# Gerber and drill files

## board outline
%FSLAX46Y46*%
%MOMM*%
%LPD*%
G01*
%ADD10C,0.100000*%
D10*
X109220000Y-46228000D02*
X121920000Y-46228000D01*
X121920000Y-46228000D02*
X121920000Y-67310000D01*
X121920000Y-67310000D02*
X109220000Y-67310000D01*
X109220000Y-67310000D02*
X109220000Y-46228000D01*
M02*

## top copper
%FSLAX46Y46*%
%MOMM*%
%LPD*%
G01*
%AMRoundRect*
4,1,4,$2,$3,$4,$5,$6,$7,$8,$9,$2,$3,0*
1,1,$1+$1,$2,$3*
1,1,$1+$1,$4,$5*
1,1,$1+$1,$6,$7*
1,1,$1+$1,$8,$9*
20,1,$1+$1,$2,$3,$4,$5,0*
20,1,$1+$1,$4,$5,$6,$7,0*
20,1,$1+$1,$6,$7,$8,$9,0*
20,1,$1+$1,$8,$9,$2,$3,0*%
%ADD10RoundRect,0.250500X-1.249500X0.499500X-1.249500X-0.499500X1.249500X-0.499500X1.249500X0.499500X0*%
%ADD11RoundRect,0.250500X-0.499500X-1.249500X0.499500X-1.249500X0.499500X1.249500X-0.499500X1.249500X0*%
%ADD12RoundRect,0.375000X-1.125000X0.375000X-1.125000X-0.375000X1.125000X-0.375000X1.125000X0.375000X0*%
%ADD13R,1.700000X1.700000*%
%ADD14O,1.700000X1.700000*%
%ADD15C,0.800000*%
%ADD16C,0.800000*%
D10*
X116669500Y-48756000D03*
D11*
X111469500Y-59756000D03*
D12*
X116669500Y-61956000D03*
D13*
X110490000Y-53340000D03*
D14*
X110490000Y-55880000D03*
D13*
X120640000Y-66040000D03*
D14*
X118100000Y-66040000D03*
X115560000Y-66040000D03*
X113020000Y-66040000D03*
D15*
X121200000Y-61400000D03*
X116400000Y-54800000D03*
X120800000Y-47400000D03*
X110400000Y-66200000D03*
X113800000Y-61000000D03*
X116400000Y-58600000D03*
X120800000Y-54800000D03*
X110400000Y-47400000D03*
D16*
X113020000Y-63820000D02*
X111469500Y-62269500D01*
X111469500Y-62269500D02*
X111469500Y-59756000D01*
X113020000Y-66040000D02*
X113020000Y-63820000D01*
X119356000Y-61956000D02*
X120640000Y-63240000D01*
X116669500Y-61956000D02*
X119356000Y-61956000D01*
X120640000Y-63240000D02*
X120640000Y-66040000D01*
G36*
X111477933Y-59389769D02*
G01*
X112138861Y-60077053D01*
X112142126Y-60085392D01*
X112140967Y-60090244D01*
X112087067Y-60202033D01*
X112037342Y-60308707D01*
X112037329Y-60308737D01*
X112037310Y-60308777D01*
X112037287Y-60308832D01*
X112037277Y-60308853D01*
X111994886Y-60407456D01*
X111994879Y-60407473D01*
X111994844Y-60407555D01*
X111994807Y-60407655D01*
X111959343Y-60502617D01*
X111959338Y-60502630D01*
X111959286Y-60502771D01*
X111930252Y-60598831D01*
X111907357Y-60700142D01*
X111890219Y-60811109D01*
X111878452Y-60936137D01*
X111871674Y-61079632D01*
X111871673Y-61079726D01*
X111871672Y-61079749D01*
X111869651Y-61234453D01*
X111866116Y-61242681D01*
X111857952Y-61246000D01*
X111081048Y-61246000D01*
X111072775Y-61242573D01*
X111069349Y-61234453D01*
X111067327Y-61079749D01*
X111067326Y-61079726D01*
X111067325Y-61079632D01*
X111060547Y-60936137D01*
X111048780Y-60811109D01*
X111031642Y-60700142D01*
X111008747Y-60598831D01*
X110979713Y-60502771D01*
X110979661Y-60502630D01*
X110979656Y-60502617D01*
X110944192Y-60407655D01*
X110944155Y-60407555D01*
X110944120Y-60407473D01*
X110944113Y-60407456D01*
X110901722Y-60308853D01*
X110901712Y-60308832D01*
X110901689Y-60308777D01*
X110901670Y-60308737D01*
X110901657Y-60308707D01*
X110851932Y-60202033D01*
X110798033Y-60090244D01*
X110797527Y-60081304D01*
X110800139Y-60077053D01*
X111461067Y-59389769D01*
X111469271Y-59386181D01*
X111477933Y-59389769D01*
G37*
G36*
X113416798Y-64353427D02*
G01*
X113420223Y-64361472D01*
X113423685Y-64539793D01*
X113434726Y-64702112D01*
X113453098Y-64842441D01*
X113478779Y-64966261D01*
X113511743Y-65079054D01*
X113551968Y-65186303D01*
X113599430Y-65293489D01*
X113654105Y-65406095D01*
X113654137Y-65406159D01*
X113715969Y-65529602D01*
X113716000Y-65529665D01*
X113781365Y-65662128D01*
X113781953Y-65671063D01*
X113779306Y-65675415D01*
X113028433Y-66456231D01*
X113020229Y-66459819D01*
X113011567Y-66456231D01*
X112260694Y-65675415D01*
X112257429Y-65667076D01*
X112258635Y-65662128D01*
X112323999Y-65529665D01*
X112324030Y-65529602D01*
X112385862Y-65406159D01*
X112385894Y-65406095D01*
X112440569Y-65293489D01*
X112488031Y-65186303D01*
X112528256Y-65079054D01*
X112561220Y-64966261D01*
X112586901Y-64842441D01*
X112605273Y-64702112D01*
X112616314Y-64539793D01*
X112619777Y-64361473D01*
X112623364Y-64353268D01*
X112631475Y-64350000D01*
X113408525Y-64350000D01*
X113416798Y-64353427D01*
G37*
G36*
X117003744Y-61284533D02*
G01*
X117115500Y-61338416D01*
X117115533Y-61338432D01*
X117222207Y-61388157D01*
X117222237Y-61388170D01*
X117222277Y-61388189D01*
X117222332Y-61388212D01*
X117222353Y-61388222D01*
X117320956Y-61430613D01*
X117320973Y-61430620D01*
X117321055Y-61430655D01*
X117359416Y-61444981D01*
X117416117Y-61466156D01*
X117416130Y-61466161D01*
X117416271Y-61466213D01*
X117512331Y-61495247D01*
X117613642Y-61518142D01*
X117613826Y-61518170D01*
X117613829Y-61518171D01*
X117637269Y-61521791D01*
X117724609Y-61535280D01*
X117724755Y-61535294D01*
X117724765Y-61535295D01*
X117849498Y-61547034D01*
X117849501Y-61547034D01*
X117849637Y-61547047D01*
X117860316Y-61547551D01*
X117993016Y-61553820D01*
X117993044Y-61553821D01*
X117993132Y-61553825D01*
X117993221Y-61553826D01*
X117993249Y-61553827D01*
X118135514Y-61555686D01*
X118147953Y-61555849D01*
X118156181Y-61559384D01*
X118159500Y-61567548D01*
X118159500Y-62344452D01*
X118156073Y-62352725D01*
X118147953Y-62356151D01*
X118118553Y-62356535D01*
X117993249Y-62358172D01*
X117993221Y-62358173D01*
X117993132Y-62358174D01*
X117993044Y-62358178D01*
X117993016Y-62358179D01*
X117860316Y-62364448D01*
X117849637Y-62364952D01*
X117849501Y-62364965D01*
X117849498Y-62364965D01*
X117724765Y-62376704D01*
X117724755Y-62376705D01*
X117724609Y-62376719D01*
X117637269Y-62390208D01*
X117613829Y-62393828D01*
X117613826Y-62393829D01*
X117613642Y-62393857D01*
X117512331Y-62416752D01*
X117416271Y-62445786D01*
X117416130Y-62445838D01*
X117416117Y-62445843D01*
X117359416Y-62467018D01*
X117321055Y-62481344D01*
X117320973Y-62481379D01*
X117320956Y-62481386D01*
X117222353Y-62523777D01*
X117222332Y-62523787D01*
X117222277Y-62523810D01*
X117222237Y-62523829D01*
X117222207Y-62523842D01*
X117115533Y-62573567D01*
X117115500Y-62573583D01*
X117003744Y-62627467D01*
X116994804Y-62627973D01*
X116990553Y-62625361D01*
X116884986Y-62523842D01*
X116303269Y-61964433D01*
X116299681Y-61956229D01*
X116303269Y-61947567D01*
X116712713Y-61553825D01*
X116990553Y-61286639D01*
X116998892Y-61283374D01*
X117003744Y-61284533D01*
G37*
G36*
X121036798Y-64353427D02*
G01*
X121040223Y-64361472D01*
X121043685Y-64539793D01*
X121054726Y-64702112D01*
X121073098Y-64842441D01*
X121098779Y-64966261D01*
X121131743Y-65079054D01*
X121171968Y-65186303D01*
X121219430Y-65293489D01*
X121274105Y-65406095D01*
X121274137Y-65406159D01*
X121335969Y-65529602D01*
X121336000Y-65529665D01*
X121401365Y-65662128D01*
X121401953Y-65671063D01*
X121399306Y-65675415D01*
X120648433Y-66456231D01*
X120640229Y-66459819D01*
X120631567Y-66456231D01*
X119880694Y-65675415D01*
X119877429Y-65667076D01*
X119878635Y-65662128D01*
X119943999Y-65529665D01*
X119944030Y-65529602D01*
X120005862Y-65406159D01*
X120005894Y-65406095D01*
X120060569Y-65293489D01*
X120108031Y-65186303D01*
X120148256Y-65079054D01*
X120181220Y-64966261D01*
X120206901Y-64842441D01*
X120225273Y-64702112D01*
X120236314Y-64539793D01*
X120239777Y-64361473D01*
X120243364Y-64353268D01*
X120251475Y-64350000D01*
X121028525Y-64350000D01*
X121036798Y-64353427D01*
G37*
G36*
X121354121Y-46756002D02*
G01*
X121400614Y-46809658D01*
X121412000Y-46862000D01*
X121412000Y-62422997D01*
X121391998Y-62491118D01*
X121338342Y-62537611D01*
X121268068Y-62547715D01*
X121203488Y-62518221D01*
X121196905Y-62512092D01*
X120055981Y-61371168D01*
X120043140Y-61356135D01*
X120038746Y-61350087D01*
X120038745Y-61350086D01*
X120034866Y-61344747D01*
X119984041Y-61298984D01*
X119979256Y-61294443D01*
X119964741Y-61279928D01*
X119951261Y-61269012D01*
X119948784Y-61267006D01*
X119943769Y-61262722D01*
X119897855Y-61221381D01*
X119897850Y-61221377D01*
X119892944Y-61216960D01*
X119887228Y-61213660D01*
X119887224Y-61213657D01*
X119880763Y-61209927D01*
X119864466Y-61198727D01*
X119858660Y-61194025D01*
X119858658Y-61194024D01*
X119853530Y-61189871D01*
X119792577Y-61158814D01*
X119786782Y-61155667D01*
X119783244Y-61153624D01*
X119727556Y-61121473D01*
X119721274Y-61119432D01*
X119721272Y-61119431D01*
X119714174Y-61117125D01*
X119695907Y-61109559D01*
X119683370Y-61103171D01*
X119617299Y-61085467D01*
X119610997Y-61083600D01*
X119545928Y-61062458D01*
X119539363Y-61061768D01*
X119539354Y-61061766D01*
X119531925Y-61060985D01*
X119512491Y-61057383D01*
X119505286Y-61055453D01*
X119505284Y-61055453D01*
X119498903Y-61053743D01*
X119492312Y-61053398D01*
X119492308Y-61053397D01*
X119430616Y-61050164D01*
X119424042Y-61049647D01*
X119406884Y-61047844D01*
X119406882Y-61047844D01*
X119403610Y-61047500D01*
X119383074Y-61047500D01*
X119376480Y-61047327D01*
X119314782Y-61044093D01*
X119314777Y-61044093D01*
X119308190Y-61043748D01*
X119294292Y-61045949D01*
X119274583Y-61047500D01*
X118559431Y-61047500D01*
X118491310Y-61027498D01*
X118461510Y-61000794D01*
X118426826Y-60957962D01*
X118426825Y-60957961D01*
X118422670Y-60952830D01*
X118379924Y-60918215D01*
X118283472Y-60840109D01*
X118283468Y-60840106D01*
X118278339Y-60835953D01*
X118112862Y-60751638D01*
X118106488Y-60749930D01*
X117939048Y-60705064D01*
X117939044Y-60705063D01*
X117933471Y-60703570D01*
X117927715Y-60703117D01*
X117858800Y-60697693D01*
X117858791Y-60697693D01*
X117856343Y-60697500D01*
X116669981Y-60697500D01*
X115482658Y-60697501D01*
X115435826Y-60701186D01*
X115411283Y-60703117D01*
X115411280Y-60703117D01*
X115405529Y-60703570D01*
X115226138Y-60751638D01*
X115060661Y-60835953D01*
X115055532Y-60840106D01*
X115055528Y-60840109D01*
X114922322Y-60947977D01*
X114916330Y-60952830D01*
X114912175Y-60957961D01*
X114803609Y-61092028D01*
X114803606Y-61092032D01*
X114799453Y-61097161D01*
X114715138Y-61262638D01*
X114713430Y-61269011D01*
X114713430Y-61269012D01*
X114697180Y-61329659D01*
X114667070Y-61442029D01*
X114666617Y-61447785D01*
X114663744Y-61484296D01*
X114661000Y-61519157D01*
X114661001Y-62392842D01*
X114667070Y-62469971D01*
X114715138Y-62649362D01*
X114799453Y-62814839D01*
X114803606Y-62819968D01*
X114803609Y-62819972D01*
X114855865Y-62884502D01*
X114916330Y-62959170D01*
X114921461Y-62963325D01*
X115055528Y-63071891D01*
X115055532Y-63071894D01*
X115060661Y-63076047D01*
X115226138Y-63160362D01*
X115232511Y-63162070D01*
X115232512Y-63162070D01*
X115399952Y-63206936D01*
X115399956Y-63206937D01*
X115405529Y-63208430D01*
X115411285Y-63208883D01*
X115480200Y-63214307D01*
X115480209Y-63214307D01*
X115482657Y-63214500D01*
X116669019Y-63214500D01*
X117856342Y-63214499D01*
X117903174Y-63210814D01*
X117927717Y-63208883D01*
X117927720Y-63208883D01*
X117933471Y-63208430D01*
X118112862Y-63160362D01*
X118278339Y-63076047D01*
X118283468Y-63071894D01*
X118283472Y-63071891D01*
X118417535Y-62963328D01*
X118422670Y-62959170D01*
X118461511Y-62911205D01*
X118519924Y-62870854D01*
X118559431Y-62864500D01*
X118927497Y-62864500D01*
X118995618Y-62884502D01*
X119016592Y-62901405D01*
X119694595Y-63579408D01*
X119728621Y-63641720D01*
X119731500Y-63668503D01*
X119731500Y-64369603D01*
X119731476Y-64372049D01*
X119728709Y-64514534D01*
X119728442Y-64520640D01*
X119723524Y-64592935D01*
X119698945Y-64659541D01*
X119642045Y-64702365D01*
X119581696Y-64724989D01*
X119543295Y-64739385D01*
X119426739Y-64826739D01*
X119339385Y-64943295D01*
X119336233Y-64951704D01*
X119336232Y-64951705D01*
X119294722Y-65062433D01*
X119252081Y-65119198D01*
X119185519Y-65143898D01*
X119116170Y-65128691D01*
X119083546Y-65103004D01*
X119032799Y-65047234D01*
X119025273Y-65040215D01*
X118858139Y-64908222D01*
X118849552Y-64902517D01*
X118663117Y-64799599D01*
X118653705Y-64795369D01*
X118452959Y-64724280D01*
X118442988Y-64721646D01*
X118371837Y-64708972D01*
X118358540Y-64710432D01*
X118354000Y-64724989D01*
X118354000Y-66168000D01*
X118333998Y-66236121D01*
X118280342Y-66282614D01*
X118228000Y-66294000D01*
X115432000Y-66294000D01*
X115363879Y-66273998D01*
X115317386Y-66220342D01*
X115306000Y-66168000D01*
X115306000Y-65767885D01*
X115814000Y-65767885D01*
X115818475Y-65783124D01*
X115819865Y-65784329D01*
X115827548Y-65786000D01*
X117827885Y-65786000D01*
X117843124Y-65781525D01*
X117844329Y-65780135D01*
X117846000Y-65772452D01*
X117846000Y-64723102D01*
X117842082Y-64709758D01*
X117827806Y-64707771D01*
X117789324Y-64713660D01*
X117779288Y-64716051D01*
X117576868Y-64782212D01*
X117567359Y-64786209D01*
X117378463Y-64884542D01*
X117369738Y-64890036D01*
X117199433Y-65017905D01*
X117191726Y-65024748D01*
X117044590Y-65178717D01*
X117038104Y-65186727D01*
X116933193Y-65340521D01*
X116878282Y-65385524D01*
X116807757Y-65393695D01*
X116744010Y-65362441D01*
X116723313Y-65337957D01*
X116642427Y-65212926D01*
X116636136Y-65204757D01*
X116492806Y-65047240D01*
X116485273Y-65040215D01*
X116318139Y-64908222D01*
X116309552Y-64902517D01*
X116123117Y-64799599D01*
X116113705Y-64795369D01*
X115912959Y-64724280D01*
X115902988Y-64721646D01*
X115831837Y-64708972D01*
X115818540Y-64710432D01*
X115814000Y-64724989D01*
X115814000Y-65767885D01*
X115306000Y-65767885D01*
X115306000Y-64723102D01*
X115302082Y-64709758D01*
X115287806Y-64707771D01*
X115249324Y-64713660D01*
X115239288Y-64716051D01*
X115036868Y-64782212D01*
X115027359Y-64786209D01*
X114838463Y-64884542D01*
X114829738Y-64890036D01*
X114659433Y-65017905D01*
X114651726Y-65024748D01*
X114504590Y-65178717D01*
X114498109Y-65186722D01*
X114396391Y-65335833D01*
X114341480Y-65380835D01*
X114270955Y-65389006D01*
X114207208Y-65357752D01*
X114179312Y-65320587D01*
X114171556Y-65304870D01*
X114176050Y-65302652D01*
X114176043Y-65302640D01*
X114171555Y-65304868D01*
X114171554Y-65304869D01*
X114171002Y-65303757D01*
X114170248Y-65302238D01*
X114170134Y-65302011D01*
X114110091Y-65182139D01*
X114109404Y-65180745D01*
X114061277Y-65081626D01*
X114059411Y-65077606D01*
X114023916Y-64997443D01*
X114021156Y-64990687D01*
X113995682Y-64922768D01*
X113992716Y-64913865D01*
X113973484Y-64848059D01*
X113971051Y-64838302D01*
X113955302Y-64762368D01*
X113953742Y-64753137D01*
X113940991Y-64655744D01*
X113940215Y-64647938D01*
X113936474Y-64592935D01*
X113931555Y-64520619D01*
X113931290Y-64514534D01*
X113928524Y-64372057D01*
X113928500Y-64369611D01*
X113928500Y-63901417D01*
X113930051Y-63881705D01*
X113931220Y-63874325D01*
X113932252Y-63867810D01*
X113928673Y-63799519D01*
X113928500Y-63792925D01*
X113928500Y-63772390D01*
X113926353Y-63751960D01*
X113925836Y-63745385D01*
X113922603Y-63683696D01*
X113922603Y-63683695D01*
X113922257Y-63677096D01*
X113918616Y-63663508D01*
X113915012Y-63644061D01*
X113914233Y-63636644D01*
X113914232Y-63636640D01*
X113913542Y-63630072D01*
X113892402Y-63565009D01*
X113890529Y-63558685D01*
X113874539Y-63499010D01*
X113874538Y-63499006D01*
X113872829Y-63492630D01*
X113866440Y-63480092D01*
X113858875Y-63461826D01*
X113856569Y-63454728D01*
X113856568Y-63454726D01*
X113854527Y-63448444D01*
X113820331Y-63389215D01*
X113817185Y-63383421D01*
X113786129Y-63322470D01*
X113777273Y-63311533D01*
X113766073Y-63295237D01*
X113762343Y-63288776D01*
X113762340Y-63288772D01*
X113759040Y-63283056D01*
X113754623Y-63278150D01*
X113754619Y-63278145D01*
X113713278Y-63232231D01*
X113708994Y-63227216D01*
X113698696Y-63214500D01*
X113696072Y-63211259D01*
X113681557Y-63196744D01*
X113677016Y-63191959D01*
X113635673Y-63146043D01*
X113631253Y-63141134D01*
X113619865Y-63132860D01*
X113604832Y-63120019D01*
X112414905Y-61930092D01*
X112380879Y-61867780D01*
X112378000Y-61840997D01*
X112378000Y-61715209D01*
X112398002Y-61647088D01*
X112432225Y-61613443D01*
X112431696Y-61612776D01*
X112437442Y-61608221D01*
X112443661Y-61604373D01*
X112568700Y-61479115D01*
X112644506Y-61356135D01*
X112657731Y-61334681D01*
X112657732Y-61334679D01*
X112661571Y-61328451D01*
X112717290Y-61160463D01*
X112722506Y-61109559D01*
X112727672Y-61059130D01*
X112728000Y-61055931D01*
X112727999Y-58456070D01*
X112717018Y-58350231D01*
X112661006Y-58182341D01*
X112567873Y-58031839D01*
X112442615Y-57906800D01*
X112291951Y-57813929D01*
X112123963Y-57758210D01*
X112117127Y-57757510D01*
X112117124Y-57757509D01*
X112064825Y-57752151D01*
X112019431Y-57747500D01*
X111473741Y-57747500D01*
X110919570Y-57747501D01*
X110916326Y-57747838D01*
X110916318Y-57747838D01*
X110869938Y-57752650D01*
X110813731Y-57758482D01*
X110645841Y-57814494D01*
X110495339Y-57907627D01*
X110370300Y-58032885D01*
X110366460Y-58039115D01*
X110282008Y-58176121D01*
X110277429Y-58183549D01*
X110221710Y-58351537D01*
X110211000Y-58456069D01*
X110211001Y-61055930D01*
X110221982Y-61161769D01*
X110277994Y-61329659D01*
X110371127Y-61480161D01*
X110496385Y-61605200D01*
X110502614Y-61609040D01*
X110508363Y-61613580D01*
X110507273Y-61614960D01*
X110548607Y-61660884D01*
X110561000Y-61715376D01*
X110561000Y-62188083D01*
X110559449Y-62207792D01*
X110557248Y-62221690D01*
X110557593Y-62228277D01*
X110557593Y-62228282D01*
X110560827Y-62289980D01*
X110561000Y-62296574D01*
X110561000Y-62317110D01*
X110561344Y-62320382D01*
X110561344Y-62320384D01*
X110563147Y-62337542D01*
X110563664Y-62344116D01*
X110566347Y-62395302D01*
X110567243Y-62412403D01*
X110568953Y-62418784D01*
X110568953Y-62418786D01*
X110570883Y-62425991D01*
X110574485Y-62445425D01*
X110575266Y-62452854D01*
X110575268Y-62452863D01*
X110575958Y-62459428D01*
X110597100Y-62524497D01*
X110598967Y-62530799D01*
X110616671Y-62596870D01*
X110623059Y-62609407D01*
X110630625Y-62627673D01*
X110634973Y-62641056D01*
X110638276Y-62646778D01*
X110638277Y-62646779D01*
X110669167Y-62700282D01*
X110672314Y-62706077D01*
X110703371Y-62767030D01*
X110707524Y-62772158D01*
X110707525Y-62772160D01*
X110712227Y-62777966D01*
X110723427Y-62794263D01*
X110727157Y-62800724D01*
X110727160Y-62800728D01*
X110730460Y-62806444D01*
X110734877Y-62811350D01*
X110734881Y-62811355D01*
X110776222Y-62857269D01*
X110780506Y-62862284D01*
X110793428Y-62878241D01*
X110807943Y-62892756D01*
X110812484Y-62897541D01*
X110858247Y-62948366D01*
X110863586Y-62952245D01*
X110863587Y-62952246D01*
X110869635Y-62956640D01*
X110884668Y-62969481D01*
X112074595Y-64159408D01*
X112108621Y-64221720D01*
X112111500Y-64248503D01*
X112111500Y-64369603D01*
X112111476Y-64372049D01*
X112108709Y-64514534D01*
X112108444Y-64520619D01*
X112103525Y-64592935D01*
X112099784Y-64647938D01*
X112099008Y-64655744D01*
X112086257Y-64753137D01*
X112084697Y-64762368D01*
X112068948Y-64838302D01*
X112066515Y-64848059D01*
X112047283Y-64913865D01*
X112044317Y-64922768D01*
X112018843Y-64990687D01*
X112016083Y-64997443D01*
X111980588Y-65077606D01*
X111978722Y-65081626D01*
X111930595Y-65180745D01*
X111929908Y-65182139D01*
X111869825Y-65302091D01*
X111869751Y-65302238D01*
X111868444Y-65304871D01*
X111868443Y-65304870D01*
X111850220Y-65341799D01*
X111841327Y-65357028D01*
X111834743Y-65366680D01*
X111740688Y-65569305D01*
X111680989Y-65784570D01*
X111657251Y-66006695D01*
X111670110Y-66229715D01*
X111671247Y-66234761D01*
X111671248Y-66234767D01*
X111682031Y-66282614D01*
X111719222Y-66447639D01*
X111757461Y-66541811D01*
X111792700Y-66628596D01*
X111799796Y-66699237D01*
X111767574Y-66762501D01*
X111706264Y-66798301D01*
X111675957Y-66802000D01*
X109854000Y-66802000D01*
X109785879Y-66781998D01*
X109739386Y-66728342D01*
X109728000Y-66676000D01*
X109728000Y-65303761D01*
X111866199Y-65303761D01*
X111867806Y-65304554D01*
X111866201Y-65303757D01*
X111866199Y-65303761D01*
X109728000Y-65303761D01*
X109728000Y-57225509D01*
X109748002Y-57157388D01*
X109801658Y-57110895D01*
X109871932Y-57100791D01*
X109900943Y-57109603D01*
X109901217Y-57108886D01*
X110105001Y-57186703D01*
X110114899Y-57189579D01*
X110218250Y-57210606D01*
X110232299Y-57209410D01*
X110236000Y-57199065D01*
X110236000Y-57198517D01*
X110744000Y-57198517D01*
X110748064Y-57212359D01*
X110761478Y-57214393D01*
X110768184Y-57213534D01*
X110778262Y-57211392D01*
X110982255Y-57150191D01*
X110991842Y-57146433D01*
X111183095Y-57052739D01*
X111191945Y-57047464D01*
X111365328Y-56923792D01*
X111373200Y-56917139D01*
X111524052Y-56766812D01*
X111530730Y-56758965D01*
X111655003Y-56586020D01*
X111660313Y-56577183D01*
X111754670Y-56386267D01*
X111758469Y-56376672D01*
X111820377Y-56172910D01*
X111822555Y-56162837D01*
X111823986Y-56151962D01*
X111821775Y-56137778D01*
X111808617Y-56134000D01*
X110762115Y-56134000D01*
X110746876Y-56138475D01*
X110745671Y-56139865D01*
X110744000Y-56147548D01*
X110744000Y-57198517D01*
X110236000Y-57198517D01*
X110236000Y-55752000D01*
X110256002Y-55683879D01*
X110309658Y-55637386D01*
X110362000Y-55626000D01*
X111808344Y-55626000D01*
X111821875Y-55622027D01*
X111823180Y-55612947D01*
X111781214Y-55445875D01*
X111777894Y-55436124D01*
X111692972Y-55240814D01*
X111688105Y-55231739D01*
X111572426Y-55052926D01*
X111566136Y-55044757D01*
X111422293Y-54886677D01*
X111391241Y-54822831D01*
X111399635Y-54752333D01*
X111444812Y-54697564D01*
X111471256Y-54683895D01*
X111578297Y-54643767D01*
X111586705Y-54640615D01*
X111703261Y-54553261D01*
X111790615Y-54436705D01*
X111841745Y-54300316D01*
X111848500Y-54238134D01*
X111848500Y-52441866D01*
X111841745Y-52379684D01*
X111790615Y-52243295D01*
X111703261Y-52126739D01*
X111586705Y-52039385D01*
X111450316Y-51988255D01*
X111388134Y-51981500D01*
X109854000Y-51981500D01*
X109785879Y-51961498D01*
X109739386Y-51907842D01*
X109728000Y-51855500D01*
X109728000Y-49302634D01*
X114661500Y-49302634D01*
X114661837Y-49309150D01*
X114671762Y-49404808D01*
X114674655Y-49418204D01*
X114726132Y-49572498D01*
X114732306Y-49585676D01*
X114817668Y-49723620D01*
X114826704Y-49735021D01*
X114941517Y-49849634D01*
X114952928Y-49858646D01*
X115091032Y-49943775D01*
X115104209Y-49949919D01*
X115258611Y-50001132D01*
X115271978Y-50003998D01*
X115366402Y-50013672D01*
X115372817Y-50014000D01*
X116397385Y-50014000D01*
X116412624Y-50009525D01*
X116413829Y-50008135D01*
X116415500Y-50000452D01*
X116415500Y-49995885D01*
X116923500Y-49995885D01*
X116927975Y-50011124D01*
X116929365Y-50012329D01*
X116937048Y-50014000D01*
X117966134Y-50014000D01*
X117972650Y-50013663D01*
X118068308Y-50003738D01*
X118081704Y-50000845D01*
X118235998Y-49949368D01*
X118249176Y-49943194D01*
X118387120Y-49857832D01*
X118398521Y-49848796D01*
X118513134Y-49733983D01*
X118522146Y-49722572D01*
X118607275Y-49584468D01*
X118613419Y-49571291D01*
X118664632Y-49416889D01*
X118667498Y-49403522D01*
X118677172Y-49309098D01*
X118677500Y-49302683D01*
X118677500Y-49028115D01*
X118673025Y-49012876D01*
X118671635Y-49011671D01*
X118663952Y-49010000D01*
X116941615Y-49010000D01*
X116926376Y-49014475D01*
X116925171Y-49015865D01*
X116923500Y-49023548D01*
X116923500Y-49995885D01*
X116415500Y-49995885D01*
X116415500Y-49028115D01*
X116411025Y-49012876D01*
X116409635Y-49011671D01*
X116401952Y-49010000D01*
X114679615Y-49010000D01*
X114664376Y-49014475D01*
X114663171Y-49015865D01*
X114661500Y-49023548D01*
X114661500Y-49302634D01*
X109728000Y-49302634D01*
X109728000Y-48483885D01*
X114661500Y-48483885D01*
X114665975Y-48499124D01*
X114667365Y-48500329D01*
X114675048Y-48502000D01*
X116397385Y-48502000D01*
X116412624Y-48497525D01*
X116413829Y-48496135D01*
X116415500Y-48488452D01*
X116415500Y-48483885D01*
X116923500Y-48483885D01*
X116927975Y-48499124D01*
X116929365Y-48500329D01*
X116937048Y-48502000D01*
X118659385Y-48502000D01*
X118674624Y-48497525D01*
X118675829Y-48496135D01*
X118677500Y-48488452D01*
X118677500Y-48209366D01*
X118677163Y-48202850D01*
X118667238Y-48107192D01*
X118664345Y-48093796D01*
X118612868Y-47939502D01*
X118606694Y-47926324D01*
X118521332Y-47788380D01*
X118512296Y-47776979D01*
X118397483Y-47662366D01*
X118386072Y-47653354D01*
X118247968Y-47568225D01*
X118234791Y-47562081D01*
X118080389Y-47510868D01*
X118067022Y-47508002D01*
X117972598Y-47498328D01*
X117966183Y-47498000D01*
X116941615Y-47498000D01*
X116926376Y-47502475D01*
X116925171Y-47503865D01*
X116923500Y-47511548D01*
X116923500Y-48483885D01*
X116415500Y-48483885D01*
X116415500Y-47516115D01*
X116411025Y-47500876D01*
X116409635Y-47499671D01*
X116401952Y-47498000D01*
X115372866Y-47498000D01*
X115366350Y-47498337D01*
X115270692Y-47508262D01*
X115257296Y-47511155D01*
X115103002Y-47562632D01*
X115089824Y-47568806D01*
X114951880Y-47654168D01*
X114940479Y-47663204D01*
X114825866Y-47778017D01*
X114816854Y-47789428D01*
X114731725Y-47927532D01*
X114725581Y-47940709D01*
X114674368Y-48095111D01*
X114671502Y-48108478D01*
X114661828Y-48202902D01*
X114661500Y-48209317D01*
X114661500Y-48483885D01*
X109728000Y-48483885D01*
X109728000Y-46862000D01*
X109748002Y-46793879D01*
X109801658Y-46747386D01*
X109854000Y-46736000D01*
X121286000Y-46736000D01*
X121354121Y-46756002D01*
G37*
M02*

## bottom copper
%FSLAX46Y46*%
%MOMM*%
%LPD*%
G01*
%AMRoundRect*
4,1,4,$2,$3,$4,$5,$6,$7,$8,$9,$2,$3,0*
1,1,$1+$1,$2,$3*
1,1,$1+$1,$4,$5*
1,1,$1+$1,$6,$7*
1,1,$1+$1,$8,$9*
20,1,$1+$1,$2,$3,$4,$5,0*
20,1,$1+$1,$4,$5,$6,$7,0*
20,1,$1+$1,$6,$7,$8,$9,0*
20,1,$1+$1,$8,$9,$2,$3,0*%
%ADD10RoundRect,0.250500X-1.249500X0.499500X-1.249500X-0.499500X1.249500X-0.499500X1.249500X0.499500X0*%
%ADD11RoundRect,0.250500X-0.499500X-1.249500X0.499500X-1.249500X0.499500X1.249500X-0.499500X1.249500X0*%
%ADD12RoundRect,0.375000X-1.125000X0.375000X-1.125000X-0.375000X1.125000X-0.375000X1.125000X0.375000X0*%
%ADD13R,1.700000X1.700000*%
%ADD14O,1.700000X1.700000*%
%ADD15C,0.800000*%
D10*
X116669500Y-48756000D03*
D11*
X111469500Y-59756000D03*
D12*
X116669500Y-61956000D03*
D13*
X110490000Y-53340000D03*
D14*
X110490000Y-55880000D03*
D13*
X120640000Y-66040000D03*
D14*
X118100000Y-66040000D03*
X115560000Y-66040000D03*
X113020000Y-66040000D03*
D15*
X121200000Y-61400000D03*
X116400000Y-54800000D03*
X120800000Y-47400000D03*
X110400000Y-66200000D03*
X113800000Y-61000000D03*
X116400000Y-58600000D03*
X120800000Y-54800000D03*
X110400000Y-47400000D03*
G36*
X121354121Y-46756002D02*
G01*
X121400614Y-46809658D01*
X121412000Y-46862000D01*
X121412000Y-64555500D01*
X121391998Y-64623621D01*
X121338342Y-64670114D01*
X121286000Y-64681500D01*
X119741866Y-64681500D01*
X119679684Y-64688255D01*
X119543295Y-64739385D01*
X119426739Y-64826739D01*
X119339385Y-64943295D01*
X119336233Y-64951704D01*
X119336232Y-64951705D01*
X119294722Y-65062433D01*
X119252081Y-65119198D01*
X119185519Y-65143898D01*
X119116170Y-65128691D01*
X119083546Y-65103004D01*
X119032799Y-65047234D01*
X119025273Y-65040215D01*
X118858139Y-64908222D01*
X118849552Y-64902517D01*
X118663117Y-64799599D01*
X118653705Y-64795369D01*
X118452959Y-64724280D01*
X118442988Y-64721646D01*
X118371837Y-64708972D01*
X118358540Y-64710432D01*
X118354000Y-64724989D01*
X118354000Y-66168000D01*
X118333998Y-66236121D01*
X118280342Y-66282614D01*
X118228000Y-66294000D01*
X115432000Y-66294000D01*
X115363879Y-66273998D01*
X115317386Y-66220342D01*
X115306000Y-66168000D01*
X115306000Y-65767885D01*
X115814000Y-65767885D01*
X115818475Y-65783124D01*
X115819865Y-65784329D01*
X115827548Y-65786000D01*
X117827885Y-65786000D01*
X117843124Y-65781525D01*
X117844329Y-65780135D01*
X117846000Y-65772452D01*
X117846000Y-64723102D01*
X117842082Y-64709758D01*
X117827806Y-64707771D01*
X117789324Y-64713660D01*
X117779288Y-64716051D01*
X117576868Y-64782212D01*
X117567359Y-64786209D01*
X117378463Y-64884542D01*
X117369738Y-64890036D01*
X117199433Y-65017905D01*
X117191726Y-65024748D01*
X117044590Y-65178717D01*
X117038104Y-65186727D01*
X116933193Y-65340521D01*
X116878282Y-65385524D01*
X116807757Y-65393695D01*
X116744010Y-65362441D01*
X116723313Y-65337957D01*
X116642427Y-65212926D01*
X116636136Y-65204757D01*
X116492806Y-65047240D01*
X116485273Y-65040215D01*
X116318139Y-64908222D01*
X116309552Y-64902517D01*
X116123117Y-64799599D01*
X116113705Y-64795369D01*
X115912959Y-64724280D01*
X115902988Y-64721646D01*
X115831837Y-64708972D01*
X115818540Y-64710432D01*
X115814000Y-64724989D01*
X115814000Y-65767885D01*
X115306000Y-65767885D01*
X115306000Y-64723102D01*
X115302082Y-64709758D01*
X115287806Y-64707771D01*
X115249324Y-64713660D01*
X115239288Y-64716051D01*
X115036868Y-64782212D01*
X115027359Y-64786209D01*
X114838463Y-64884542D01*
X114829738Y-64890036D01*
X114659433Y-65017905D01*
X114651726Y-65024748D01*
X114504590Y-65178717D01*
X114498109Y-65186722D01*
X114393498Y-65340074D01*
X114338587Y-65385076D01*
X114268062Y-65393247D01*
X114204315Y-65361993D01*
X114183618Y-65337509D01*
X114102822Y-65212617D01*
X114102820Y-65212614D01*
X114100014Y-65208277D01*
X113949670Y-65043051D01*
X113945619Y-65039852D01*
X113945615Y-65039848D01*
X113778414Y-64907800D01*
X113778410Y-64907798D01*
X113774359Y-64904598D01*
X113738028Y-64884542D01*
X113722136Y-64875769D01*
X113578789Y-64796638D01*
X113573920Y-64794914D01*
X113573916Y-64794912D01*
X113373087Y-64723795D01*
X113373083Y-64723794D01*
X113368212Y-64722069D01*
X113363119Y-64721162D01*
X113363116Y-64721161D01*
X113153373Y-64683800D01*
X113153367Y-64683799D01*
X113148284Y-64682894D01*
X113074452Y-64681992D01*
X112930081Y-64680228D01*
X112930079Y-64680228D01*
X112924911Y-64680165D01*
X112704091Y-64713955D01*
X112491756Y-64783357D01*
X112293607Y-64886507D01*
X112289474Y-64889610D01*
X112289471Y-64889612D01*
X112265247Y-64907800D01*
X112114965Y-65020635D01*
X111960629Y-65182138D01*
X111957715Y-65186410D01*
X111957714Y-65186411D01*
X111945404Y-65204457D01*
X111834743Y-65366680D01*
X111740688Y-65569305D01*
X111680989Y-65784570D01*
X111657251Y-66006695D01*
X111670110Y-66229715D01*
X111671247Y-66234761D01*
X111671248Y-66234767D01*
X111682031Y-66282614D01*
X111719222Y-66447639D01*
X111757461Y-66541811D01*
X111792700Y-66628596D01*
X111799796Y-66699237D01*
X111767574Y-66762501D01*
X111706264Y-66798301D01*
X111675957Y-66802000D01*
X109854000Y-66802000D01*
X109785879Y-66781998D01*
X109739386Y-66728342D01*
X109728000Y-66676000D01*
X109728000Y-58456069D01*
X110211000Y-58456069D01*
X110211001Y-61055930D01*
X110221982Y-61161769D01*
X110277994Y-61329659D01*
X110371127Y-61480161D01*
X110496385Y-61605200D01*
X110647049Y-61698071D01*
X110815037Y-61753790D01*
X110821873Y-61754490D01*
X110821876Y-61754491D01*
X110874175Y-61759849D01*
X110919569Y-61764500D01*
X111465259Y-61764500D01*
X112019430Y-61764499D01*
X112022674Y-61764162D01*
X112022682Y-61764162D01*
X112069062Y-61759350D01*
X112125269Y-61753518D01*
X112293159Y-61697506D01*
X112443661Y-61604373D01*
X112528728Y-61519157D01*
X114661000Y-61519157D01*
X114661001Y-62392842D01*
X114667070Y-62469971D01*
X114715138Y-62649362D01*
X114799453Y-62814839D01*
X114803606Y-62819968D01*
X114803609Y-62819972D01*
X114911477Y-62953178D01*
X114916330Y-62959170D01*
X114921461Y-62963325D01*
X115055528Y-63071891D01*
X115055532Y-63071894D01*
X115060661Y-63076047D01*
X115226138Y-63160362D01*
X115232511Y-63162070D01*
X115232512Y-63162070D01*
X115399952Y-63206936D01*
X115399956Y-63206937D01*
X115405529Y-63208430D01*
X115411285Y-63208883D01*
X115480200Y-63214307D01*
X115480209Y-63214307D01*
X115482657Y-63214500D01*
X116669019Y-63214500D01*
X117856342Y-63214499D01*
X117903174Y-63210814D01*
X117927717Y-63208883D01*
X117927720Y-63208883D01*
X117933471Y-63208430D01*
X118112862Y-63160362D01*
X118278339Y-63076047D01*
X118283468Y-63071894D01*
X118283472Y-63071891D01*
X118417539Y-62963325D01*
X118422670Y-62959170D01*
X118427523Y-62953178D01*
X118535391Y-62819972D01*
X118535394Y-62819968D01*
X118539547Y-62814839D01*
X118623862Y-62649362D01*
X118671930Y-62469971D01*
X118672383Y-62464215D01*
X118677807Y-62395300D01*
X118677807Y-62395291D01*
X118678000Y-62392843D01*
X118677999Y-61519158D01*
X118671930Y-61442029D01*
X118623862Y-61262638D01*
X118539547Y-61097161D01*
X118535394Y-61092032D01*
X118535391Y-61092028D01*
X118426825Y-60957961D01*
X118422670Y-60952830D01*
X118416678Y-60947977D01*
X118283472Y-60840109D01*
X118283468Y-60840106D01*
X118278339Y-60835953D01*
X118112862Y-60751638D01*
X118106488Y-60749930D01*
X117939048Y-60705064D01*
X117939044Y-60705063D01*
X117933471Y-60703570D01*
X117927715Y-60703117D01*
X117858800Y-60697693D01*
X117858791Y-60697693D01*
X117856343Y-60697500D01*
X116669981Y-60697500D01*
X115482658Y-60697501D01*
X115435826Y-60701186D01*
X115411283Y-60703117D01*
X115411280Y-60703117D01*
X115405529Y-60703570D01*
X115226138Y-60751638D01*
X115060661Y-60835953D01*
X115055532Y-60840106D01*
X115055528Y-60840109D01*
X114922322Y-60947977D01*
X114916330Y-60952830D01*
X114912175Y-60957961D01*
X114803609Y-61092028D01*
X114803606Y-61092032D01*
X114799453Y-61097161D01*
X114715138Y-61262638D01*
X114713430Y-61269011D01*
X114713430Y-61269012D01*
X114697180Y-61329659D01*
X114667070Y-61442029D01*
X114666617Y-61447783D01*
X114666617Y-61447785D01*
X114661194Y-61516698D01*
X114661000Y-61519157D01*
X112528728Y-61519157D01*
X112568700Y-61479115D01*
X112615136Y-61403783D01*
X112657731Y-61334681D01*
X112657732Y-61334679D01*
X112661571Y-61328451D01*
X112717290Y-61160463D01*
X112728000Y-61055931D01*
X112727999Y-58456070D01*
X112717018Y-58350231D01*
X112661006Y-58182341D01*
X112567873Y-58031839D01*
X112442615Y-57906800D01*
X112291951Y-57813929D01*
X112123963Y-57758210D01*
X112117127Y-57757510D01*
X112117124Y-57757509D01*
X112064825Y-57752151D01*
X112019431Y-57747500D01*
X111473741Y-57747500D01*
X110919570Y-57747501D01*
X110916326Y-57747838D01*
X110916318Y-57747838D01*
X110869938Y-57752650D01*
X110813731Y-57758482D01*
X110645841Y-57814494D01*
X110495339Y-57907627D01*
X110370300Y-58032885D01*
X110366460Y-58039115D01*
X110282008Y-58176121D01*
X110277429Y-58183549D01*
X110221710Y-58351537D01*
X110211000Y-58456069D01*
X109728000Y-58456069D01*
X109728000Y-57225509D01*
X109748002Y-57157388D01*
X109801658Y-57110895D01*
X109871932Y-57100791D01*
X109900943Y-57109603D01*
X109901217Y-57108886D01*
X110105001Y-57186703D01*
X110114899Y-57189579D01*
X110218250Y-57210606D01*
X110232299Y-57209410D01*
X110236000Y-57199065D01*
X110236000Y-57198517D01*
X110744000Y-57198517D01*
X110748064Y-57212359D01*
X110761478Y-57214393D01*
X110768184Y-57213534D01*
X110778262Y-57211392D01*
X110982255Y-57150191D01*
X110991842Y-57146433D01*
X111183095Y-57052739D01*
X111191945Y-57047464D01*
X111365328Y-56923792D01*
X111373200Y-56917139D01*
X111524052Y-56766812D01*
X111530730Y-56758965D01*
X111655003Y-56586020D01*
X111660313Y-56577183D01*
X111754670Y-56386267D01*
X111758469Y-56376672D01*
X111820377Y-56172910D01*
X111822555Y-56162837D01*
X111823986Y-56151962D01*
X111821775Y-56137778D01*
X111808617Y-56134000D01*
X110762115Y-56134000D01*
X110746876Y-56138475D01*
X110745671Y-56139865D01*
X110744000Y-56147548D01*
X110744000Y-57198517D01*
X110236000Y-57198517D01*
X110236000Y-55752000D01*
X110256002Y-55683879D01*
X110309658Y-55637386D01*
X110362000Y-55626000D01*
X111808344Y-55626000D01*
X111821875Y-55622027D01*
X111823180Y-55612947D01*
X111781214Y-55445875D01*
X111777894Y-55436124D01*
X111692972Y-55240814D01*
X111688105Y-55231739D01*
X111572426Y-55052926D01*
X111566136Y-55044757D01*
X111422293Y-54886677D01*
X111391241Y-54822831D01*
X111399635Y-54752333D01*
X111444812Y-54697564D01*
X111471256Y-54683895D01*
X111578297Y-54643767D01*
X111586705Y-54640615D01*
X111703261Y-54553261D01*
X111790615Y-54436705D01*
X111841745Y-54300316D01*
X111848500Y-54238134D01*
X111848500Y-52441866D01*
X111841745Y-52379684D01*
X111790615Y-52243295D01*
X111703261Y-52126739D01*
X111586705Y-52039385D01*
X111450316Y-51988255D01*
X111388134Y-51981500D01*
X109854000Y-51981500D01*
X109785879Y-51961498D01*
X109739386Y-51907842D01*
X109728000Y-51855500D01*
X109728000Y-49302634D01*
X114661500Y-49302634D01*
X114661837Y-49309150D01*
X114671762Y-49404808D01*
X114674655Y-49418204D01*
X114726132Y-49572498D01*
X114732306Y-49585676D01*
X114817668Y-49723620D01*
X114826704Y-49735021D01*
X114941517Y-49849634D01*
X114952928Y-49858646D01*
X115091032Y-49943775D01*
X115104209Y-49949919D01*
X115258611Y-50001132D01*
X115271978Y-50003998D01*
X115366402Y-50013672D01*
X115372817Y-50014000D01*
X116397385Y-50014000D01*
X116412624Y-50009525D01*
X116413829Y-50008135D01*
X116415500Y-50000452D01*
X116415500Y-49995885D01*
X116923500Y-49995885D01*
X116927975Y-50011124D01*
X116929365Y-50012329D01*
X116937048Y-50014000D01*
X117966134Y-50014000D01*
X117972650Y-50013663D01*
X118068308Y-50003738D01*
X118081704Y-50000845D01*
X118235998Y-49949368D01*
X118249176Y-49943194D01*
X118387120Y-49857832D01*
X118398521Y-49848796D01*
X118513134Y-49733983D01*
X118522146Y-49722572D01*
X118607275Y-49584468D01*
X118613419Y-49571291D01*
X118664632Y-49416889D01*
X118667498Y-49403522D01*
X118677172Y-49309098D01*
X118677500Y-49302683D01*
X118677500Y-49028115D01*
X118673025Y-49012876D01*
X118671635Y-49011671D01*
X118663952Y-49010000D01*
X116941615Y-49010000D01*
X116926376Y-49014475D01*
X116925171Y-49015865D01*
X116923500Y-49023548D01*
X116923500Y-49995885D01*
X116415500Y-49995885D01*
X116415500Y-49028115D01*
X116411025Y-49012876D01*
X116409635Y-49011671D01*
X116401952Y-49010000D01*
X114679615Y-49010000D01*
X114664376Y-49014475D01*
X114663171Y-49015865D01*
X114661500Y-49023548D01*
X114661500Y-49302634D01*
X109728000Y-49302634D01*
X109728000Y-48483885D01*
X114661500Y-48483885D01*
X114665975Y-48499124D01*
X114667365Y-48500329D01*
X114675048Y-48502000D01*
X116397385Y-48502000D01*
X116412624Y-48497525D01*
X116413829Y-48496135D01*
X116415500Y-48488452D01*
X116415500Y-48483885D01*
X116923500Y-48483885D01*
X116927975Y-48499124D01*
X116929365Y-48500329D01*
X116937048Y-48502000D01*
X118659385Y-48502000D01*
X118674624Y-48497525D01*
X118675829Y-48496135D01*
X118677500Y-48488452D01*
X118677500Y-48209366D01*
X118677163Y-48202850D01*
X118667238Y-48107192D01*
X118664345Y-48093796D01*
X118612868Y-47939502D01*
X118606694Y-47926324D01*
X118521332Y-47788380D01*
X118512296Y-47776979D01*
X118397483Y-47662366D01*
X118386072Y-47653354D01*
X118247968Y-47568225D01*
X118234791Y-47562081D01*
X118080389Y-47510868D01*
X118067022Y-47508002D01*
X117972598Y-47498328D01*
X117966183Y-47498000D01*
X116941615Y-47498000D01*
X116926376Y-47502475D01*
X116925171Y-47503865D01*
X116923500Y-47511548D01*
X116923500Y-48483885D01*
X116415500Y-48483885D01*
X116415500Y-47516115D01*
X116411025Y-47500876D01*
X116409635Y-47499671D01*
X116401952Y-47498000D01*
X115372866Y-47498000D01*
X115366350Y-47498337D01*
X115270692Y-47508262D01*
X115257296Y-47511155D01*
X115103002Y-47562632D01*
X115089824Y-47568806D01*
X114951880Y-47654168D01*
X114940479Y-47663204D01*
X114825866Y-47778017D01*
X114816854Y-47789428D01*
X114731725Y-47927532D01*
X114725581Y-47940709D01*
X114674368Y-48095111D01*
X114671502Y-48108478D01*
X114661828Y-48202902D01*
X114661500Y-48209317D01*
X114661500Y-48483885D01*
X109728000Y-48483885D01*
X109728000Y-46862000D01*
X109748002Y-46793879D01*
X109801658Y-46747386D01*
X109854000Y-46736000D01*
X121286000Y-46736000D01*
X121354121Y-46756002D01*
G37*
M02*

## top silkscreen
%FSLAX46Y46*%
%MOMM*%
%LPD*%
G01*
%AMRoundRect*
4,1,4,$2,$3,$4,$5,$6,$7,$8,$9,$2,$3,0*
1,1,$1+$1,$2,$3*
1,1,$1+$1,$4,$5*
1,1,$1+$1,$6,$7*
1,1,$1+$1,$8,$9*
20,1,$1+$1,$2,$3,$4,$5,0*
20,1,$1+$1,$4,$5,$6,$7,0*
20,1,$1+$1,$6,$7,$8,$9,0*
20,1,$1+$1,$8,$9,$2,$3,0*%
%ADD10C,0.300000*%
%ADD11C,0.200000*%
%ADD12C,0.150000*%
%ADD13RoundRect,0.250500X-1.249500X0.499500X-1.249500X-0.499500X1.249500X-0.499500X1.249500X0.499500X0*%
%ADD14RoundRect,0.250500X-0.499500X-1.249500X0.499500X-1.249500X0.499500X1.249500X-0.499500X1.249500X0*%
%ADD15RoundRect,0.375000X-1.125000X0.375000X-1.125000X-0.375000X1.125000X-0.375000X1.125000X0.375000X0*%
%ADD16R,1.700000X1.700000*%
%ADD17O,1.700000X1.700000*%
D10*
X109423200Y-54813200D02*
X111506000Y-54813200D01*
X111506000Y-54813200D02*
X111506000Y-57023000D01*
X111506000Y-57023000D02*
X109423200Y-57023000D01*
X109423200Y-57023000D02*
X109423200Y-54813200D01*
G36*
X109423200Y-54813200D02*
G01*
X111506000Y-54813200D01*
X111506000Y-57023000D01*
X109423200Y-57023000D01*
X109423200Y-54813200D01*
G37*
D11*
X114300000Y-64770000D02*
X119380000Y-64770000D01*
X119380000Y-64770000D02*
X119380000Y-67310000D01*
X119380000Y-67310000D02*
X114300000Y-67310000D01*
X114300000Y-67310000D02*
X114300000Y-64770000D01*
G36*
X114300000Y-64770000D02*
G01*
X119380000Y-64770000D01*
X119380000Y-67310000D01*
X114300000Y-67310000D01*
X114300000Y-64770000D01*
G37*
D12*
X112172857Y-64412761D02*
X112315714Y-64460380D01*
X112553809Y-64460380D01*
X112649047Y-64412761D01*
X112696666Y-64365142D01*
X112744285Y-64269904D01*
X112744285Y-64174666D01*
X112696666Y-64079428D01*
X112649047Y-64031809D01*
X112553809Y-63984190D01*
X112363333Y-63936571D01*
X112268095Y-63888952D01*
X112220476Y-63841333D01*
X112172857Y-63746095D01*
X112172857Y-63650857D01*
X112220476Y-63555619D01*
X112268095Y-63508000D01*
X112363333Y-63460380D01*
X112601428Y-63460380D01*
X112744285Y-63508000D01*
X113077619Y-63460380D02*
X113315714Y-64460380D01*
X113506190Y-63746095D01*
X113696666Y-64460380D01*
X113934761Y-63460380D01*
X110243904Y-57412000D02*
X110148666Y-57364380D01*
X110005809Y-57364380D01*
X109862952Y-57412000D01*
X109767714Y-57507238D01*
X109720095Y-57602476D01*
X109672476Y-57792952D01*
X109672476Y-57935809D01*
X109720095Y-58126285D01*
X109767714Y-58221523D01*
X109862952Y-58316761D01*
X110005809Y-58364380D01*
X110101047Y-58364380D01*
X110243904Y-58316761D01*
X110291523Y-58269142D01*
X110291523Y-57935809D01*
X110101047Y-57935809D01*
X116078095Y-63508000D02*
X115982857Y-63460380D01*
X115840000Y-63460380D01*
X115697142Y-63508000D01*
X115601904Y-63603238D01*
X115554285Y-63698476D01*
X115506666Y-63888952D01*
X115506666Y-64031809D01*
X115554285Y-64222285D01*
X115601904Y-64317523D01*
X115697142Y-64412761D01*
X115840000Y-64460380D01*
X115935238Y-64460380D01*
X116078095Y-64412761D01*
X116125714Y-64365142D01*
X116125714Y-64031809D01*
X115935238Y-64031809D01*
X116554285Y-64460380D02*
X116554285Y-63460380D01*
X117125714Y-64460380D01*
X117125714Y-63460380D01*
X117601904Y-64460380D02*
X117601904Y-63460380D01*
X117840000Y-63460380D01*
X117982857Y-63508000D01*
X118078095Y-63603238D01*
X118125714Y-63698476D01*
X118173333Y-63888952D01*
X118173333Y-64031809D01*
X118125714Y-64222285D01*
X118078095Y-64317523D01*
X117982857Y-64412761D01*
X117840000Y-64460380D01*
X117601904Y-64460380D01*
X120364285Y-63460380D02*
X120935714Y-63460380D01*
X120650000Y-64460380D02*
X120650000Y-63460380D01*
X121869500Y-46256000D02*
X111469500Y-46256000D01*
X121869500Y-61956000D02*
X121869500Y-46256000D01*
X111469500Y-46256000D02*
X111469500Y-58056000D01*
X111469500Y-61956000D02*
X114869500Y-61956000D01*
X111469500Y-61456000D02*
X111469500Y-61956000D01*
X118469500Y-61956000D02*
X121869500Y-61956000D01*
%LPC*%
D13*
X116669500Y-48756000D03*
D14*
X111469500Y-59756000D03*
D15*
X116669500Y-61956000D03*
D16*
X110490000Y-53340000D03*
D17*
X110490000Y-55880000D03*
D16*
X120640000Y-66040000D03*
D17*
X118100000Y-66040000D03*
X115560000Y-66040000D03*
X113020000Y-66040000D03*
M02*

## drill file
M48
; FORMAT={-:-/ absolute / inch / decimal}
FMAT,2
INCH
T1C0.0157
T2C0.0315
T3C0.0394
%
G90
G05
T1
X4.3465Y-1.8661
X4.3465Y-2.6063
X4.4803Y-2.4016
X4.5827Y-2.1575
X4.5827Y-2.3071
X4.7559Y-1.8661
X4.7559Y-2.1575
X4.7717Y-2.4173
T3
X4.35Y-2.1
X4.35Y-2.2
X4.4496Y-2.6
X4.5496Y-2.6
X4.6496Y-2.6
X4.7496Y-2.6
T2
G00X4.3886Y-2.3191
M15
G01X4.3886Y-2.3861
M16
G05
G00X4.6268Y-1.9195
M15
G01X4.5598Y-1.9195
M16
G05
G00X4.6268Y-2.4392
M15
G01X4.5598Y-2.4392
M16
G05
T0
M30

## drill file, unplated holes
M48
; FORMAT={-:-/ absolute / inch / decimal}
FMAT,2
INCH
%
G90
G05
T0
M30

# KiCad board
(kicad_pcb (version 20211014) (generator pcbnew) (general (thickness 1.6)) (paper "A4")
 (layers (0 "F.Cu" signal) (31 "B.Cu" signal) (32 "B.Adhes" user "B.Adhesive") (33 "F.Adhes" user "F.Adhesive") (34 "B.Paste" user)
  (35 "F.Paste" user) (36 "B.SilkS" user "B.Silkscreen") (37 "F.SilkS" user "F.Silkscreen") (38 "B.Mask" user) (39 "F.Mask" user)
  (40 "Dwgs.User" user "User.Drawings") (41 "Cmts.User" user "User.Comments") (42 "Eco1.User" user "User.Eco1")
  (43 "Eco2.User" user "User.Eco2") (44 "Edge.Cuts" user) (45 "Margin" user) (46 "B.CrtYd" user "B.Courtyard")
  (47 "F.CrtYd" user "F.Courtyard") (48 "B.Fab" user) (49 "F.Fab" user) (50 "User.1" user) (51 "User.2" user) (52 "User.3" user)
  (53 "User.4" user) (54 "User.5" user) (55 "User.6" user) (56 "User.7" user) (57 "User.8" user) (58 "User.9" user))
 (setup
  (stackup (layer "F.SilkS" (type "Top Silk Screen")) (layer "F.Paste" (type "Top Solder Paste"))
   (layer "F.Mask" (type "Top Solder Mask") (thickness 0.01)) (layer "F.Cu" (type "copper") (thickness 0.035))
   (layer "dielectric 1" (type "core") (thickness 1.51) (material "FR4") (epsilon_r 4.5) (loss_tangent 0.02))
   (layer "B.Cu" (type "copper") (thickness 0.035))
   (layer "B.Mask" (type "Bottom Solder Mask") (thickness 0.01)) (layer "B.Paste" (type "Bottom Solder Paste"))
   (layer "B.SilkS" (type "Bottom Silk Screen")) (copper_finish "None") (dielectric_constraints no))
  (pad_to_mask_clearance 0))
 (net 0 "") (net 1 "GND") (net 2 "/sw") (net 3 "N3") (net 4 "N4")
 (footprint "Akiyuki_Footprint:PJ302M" (layer "F.Cu") (at 116.6695 46.256 -90)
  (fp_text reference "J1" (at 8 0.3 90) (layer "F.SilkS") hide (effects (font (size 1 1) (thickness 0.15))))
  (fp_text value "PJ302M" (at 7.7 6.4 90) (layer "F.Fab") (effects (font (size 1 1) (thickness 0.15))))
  (fp_line (start 0 -5.2) (end 0 5.2) (layer "F.SilkS") (width 0.15))
  (fp_line (start 15.7 -5.2) (end 0 -5.2) (layer "F.SilkS") (width 0.15))
  (fp_line (start 0 5.2) (end 11.8 5.2) (layer "F.SilkS") (width 0.15))
  (fp_line (start 15.7 5.2) (end 15.7 1.8) (layer "F.SilkS") (width 0.15))
  (fp_line (start 15.2 5.2) (end 15.7 5.2) (layer "F.SilkS") (width 0.15))
  (fp_line (start 15.7 -1.8) (end 15.7 -5.2) (layer "F.SilkS") (width 0.15))
  (pad "1" thru_hole roundrect locked (at 2.5 0 270) (size 1.5 3) (drill oval 0.8 2.5) (layers *.Cu *.Mask) (roundrect_rratio 0.167)
   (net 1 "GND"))
  (pad "2" thru_hole roundrect locked (at 13.5 5.2) (size 1.5 3) (drill oval 0.8 2.5) (layers *.Cu *.Mask) (roundrect_rratio 0.167)
   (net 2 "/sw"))
  (pad "3" thru_hole roundrect locked (at 15.7 0 270) (size 1.5 3) (drill oval 0.8 2.5) (layers *.Cu *.Mask) (roundrect_rratio 0.25)
   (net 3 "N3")))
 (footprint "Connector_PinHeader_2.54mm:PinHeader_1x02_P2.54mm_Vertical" (layer "B.Cu") (at 110.49 53.34 180)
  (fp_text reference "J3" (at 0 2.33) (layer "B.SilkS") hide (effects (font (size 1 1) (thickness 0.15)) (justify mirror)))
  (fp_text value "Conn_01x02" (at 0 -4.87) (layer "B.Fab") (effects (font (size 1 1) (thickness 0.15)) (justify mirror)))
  (pad "1" thru_hole rect (at 0 0 180) (size 1.7 1.7) (drill 1) (layers *.Cu *.Mask) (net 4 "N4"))
  (pad "2" thru_hole oval (at 0 -2.54 180) (size 1.7 1.7) (drill 1) (layers *.Cu *.Mask) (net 1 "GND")))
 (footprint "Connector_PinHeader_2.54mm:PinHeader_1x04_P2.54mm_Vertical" (layer "B.Cu") (at 120.64 66.04 90)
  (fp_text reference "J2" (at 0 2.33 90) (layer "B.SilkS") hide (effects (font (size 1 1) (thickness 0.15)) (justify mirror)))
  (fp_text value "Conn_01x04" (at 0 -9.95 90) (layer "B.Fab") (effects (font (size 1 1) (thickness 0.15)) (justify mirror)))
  (pad "1" thru_hole rect (at 0 0 90) (size 1.7 1.7) (drill 1) (layers *.Cu *.Mask) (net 3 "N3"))
  (pad "2" thru_hole oval (at 0 -2.54 90) (size 1.7 1.7) (drill 1) (layers *.Cu *.Mask) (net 1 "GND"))
  (pad "3" thru_hole oval (at 0 -5.08 90) (size 1.7 1.7) (drill 1) (layers *.Cu *.Mask) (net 1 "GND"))
  (pad "4" thru_hole oval (at 0 -7.62 90) (size 1.7 1.7) (drill 1) (layers *.Cu *.Mask) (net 2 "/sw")))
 (gr_rect (start 109.4232 54.8132) (end 111.506 57.023) (layer "F.SilkS") (width 0.3) (fill solid))
 (gr_rect (start 114.3 64.77) (end 119.38 67.31) (layer "F.SilkS") (width 0.2) (fill solid))
 (gr_rect (start 109.22 46.228) (end 121.92 67.31) (layer "Edge.Cuts") (width 0.1) (fill none))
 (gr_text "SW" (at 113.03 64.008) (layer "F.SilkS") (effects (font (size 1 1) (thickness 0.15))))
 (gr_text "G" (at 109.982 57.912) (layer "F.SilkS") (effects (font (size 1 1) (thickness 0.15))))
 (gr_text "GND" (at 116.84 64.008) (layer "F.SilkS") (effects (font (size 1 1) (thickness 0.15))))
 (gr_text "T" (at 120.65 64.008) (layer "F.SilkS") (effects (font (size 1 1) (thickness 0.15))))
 (via (at 121.2 61.4) (size 0.8) (drill 0.4) (layers "F.Cu" "B.Cu") (free) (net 1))
 (via (at 116.4 54.8) (size 0.8) (drill 0.4) (layers "F.Cu" "B.Cu") (free) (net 1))
 (via (at 120.8 47.4) (size 0.8) (drill 0.4) (layers "F.Cu" "B.Cu") (free) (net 1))
 (via (at 110.4 66.2) (size 0.8) (drill 0.4) (layers "F.Cu" "B.Cu") (free) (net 1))
 (via (at 113.8 61) (size 0.8) (drill 0.4) (layers "F.Cu" "B.Cu") (free) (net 1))
 (via (at 116.4 58.6) (size 0.8) (drill 0.4) (layers "F.Cu" "B.Cu") (free) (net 1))
 (via (at 120.8 54.8) (size 0.8) (drill 0.4) (layers "F.Cu" "B.Cu") (free) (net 1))
 (via (at 110.4 47.4) (size 0.8) (drill 0.4) (layers "F.Cu" "B.Cu") (free) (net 1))
 (segment (start 113.02 63.82) (end 111.4695 62.2695) (width 0.8) (layer "F.Cu") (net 2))
 (segment (start 111.4695 62.2695) (end 111.4695 59.756) (width 0.8) (layer "F.Cu") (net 2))
 (segment (start 113.02 66.04) (end 113.02 63.82) (width 0.8) (layer "F.Cu") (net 2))
 (segment (start 119.356 61.956) (end 120.64 63.24) (width 0.8) (layer "F.Cu") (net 3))
 (segment (start 116.6695 61.956) (end 119.356 61.956) (width 0.8) (layer "F.Cu") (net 3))
 (segment (start 120.64 63.24) (end 120.64 66.04) (width 0.8) (layer "F.Cu") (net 3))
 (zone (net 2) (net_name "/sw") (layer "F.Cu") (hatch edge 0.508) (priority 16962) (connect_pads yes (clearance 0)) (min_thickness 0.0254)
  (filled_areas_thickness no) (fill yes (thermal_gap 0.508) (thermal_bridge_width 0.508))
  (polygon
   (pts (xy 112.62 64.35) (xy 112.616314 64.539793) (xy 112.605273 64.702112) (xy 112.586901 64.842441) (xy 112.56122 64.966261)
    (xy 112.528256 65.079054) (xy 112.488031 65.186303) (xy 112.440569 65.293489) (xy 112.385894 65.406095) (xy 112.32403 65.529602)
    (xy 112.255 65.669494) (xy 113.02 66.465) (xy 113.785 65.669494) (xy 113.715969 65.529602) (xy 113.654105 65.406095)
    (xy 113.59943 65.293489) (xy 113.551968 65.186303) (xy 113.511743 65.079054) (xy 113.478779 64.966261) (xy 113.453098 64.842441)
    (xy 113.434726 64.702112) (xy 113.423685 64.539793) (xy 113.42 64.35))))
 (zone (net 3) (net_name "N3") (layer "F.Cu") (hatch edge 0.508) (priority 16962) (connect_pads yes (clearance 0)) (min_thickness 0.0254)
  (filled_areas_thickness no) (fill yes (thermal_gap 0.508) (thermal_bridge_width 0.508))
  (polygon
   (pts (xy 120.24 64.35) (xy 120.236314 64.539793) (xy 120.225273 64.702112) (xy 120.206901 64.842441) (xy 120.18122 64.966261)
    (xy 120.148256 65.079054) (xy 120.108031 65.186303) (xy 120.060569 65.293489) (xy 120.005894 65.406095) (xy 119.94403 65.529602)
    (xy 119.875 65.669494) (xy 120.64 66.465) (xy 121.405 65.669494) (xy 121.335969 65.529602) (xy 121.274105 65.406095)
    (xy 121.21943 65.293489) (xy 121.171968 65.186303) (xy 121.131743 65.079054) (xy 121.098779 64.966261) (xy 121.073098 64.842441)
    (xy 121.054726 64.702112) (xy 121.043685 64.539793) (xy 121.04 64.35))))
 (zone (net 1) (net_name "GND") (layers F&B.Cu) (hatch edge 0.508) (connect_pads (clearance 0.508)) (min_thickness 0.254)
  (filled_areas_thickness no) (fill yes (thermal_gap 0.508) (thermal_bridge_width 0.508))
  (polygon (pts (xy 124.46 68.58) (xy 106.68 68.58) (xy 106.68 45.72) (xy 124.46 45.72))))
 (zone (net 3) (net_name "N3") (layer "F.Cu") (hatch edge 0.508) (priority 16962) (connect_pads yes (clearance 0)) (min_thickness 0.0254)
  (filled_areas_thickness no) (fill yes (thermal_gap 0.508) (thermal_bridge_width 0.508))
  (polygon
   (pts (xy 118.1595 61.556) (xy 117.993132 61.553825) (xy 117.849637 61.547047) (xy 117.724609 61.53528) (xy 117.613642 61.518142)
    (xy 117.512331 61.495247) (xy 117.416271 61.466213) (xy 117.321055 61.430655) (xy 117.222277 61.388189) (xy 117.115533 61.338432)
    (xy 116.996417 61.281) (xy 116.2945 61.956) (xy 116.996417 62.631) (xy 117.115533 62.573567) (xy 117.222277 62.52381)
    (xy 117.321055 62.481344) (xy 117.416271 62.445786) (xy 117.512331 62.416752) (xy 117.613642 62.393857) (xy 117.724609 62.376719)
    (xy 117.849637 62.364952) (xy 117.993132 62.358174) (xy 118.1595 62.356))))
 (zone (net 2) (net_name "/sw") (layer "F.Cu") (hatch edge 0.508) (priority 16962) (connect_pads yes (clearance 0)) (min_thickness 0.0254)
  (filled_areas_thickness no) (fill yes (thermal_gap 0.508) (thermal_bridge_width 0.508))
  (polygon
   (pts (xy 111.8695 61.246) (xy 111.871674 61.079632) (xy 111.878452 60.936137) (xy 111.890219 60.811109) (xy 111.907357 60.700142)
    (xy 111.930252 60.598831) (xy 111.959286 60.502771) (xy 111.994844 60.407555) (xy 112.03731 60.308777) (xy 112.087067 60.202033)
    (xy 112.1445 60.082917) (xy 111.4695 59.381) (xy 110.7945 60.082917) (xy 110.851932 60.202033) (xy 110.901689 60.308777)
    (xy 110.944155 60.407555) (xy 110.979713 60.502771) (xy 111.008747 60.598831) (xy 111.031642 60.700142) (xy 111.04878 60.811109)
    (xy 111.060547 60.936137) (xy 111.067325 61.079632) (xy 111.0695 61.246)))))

